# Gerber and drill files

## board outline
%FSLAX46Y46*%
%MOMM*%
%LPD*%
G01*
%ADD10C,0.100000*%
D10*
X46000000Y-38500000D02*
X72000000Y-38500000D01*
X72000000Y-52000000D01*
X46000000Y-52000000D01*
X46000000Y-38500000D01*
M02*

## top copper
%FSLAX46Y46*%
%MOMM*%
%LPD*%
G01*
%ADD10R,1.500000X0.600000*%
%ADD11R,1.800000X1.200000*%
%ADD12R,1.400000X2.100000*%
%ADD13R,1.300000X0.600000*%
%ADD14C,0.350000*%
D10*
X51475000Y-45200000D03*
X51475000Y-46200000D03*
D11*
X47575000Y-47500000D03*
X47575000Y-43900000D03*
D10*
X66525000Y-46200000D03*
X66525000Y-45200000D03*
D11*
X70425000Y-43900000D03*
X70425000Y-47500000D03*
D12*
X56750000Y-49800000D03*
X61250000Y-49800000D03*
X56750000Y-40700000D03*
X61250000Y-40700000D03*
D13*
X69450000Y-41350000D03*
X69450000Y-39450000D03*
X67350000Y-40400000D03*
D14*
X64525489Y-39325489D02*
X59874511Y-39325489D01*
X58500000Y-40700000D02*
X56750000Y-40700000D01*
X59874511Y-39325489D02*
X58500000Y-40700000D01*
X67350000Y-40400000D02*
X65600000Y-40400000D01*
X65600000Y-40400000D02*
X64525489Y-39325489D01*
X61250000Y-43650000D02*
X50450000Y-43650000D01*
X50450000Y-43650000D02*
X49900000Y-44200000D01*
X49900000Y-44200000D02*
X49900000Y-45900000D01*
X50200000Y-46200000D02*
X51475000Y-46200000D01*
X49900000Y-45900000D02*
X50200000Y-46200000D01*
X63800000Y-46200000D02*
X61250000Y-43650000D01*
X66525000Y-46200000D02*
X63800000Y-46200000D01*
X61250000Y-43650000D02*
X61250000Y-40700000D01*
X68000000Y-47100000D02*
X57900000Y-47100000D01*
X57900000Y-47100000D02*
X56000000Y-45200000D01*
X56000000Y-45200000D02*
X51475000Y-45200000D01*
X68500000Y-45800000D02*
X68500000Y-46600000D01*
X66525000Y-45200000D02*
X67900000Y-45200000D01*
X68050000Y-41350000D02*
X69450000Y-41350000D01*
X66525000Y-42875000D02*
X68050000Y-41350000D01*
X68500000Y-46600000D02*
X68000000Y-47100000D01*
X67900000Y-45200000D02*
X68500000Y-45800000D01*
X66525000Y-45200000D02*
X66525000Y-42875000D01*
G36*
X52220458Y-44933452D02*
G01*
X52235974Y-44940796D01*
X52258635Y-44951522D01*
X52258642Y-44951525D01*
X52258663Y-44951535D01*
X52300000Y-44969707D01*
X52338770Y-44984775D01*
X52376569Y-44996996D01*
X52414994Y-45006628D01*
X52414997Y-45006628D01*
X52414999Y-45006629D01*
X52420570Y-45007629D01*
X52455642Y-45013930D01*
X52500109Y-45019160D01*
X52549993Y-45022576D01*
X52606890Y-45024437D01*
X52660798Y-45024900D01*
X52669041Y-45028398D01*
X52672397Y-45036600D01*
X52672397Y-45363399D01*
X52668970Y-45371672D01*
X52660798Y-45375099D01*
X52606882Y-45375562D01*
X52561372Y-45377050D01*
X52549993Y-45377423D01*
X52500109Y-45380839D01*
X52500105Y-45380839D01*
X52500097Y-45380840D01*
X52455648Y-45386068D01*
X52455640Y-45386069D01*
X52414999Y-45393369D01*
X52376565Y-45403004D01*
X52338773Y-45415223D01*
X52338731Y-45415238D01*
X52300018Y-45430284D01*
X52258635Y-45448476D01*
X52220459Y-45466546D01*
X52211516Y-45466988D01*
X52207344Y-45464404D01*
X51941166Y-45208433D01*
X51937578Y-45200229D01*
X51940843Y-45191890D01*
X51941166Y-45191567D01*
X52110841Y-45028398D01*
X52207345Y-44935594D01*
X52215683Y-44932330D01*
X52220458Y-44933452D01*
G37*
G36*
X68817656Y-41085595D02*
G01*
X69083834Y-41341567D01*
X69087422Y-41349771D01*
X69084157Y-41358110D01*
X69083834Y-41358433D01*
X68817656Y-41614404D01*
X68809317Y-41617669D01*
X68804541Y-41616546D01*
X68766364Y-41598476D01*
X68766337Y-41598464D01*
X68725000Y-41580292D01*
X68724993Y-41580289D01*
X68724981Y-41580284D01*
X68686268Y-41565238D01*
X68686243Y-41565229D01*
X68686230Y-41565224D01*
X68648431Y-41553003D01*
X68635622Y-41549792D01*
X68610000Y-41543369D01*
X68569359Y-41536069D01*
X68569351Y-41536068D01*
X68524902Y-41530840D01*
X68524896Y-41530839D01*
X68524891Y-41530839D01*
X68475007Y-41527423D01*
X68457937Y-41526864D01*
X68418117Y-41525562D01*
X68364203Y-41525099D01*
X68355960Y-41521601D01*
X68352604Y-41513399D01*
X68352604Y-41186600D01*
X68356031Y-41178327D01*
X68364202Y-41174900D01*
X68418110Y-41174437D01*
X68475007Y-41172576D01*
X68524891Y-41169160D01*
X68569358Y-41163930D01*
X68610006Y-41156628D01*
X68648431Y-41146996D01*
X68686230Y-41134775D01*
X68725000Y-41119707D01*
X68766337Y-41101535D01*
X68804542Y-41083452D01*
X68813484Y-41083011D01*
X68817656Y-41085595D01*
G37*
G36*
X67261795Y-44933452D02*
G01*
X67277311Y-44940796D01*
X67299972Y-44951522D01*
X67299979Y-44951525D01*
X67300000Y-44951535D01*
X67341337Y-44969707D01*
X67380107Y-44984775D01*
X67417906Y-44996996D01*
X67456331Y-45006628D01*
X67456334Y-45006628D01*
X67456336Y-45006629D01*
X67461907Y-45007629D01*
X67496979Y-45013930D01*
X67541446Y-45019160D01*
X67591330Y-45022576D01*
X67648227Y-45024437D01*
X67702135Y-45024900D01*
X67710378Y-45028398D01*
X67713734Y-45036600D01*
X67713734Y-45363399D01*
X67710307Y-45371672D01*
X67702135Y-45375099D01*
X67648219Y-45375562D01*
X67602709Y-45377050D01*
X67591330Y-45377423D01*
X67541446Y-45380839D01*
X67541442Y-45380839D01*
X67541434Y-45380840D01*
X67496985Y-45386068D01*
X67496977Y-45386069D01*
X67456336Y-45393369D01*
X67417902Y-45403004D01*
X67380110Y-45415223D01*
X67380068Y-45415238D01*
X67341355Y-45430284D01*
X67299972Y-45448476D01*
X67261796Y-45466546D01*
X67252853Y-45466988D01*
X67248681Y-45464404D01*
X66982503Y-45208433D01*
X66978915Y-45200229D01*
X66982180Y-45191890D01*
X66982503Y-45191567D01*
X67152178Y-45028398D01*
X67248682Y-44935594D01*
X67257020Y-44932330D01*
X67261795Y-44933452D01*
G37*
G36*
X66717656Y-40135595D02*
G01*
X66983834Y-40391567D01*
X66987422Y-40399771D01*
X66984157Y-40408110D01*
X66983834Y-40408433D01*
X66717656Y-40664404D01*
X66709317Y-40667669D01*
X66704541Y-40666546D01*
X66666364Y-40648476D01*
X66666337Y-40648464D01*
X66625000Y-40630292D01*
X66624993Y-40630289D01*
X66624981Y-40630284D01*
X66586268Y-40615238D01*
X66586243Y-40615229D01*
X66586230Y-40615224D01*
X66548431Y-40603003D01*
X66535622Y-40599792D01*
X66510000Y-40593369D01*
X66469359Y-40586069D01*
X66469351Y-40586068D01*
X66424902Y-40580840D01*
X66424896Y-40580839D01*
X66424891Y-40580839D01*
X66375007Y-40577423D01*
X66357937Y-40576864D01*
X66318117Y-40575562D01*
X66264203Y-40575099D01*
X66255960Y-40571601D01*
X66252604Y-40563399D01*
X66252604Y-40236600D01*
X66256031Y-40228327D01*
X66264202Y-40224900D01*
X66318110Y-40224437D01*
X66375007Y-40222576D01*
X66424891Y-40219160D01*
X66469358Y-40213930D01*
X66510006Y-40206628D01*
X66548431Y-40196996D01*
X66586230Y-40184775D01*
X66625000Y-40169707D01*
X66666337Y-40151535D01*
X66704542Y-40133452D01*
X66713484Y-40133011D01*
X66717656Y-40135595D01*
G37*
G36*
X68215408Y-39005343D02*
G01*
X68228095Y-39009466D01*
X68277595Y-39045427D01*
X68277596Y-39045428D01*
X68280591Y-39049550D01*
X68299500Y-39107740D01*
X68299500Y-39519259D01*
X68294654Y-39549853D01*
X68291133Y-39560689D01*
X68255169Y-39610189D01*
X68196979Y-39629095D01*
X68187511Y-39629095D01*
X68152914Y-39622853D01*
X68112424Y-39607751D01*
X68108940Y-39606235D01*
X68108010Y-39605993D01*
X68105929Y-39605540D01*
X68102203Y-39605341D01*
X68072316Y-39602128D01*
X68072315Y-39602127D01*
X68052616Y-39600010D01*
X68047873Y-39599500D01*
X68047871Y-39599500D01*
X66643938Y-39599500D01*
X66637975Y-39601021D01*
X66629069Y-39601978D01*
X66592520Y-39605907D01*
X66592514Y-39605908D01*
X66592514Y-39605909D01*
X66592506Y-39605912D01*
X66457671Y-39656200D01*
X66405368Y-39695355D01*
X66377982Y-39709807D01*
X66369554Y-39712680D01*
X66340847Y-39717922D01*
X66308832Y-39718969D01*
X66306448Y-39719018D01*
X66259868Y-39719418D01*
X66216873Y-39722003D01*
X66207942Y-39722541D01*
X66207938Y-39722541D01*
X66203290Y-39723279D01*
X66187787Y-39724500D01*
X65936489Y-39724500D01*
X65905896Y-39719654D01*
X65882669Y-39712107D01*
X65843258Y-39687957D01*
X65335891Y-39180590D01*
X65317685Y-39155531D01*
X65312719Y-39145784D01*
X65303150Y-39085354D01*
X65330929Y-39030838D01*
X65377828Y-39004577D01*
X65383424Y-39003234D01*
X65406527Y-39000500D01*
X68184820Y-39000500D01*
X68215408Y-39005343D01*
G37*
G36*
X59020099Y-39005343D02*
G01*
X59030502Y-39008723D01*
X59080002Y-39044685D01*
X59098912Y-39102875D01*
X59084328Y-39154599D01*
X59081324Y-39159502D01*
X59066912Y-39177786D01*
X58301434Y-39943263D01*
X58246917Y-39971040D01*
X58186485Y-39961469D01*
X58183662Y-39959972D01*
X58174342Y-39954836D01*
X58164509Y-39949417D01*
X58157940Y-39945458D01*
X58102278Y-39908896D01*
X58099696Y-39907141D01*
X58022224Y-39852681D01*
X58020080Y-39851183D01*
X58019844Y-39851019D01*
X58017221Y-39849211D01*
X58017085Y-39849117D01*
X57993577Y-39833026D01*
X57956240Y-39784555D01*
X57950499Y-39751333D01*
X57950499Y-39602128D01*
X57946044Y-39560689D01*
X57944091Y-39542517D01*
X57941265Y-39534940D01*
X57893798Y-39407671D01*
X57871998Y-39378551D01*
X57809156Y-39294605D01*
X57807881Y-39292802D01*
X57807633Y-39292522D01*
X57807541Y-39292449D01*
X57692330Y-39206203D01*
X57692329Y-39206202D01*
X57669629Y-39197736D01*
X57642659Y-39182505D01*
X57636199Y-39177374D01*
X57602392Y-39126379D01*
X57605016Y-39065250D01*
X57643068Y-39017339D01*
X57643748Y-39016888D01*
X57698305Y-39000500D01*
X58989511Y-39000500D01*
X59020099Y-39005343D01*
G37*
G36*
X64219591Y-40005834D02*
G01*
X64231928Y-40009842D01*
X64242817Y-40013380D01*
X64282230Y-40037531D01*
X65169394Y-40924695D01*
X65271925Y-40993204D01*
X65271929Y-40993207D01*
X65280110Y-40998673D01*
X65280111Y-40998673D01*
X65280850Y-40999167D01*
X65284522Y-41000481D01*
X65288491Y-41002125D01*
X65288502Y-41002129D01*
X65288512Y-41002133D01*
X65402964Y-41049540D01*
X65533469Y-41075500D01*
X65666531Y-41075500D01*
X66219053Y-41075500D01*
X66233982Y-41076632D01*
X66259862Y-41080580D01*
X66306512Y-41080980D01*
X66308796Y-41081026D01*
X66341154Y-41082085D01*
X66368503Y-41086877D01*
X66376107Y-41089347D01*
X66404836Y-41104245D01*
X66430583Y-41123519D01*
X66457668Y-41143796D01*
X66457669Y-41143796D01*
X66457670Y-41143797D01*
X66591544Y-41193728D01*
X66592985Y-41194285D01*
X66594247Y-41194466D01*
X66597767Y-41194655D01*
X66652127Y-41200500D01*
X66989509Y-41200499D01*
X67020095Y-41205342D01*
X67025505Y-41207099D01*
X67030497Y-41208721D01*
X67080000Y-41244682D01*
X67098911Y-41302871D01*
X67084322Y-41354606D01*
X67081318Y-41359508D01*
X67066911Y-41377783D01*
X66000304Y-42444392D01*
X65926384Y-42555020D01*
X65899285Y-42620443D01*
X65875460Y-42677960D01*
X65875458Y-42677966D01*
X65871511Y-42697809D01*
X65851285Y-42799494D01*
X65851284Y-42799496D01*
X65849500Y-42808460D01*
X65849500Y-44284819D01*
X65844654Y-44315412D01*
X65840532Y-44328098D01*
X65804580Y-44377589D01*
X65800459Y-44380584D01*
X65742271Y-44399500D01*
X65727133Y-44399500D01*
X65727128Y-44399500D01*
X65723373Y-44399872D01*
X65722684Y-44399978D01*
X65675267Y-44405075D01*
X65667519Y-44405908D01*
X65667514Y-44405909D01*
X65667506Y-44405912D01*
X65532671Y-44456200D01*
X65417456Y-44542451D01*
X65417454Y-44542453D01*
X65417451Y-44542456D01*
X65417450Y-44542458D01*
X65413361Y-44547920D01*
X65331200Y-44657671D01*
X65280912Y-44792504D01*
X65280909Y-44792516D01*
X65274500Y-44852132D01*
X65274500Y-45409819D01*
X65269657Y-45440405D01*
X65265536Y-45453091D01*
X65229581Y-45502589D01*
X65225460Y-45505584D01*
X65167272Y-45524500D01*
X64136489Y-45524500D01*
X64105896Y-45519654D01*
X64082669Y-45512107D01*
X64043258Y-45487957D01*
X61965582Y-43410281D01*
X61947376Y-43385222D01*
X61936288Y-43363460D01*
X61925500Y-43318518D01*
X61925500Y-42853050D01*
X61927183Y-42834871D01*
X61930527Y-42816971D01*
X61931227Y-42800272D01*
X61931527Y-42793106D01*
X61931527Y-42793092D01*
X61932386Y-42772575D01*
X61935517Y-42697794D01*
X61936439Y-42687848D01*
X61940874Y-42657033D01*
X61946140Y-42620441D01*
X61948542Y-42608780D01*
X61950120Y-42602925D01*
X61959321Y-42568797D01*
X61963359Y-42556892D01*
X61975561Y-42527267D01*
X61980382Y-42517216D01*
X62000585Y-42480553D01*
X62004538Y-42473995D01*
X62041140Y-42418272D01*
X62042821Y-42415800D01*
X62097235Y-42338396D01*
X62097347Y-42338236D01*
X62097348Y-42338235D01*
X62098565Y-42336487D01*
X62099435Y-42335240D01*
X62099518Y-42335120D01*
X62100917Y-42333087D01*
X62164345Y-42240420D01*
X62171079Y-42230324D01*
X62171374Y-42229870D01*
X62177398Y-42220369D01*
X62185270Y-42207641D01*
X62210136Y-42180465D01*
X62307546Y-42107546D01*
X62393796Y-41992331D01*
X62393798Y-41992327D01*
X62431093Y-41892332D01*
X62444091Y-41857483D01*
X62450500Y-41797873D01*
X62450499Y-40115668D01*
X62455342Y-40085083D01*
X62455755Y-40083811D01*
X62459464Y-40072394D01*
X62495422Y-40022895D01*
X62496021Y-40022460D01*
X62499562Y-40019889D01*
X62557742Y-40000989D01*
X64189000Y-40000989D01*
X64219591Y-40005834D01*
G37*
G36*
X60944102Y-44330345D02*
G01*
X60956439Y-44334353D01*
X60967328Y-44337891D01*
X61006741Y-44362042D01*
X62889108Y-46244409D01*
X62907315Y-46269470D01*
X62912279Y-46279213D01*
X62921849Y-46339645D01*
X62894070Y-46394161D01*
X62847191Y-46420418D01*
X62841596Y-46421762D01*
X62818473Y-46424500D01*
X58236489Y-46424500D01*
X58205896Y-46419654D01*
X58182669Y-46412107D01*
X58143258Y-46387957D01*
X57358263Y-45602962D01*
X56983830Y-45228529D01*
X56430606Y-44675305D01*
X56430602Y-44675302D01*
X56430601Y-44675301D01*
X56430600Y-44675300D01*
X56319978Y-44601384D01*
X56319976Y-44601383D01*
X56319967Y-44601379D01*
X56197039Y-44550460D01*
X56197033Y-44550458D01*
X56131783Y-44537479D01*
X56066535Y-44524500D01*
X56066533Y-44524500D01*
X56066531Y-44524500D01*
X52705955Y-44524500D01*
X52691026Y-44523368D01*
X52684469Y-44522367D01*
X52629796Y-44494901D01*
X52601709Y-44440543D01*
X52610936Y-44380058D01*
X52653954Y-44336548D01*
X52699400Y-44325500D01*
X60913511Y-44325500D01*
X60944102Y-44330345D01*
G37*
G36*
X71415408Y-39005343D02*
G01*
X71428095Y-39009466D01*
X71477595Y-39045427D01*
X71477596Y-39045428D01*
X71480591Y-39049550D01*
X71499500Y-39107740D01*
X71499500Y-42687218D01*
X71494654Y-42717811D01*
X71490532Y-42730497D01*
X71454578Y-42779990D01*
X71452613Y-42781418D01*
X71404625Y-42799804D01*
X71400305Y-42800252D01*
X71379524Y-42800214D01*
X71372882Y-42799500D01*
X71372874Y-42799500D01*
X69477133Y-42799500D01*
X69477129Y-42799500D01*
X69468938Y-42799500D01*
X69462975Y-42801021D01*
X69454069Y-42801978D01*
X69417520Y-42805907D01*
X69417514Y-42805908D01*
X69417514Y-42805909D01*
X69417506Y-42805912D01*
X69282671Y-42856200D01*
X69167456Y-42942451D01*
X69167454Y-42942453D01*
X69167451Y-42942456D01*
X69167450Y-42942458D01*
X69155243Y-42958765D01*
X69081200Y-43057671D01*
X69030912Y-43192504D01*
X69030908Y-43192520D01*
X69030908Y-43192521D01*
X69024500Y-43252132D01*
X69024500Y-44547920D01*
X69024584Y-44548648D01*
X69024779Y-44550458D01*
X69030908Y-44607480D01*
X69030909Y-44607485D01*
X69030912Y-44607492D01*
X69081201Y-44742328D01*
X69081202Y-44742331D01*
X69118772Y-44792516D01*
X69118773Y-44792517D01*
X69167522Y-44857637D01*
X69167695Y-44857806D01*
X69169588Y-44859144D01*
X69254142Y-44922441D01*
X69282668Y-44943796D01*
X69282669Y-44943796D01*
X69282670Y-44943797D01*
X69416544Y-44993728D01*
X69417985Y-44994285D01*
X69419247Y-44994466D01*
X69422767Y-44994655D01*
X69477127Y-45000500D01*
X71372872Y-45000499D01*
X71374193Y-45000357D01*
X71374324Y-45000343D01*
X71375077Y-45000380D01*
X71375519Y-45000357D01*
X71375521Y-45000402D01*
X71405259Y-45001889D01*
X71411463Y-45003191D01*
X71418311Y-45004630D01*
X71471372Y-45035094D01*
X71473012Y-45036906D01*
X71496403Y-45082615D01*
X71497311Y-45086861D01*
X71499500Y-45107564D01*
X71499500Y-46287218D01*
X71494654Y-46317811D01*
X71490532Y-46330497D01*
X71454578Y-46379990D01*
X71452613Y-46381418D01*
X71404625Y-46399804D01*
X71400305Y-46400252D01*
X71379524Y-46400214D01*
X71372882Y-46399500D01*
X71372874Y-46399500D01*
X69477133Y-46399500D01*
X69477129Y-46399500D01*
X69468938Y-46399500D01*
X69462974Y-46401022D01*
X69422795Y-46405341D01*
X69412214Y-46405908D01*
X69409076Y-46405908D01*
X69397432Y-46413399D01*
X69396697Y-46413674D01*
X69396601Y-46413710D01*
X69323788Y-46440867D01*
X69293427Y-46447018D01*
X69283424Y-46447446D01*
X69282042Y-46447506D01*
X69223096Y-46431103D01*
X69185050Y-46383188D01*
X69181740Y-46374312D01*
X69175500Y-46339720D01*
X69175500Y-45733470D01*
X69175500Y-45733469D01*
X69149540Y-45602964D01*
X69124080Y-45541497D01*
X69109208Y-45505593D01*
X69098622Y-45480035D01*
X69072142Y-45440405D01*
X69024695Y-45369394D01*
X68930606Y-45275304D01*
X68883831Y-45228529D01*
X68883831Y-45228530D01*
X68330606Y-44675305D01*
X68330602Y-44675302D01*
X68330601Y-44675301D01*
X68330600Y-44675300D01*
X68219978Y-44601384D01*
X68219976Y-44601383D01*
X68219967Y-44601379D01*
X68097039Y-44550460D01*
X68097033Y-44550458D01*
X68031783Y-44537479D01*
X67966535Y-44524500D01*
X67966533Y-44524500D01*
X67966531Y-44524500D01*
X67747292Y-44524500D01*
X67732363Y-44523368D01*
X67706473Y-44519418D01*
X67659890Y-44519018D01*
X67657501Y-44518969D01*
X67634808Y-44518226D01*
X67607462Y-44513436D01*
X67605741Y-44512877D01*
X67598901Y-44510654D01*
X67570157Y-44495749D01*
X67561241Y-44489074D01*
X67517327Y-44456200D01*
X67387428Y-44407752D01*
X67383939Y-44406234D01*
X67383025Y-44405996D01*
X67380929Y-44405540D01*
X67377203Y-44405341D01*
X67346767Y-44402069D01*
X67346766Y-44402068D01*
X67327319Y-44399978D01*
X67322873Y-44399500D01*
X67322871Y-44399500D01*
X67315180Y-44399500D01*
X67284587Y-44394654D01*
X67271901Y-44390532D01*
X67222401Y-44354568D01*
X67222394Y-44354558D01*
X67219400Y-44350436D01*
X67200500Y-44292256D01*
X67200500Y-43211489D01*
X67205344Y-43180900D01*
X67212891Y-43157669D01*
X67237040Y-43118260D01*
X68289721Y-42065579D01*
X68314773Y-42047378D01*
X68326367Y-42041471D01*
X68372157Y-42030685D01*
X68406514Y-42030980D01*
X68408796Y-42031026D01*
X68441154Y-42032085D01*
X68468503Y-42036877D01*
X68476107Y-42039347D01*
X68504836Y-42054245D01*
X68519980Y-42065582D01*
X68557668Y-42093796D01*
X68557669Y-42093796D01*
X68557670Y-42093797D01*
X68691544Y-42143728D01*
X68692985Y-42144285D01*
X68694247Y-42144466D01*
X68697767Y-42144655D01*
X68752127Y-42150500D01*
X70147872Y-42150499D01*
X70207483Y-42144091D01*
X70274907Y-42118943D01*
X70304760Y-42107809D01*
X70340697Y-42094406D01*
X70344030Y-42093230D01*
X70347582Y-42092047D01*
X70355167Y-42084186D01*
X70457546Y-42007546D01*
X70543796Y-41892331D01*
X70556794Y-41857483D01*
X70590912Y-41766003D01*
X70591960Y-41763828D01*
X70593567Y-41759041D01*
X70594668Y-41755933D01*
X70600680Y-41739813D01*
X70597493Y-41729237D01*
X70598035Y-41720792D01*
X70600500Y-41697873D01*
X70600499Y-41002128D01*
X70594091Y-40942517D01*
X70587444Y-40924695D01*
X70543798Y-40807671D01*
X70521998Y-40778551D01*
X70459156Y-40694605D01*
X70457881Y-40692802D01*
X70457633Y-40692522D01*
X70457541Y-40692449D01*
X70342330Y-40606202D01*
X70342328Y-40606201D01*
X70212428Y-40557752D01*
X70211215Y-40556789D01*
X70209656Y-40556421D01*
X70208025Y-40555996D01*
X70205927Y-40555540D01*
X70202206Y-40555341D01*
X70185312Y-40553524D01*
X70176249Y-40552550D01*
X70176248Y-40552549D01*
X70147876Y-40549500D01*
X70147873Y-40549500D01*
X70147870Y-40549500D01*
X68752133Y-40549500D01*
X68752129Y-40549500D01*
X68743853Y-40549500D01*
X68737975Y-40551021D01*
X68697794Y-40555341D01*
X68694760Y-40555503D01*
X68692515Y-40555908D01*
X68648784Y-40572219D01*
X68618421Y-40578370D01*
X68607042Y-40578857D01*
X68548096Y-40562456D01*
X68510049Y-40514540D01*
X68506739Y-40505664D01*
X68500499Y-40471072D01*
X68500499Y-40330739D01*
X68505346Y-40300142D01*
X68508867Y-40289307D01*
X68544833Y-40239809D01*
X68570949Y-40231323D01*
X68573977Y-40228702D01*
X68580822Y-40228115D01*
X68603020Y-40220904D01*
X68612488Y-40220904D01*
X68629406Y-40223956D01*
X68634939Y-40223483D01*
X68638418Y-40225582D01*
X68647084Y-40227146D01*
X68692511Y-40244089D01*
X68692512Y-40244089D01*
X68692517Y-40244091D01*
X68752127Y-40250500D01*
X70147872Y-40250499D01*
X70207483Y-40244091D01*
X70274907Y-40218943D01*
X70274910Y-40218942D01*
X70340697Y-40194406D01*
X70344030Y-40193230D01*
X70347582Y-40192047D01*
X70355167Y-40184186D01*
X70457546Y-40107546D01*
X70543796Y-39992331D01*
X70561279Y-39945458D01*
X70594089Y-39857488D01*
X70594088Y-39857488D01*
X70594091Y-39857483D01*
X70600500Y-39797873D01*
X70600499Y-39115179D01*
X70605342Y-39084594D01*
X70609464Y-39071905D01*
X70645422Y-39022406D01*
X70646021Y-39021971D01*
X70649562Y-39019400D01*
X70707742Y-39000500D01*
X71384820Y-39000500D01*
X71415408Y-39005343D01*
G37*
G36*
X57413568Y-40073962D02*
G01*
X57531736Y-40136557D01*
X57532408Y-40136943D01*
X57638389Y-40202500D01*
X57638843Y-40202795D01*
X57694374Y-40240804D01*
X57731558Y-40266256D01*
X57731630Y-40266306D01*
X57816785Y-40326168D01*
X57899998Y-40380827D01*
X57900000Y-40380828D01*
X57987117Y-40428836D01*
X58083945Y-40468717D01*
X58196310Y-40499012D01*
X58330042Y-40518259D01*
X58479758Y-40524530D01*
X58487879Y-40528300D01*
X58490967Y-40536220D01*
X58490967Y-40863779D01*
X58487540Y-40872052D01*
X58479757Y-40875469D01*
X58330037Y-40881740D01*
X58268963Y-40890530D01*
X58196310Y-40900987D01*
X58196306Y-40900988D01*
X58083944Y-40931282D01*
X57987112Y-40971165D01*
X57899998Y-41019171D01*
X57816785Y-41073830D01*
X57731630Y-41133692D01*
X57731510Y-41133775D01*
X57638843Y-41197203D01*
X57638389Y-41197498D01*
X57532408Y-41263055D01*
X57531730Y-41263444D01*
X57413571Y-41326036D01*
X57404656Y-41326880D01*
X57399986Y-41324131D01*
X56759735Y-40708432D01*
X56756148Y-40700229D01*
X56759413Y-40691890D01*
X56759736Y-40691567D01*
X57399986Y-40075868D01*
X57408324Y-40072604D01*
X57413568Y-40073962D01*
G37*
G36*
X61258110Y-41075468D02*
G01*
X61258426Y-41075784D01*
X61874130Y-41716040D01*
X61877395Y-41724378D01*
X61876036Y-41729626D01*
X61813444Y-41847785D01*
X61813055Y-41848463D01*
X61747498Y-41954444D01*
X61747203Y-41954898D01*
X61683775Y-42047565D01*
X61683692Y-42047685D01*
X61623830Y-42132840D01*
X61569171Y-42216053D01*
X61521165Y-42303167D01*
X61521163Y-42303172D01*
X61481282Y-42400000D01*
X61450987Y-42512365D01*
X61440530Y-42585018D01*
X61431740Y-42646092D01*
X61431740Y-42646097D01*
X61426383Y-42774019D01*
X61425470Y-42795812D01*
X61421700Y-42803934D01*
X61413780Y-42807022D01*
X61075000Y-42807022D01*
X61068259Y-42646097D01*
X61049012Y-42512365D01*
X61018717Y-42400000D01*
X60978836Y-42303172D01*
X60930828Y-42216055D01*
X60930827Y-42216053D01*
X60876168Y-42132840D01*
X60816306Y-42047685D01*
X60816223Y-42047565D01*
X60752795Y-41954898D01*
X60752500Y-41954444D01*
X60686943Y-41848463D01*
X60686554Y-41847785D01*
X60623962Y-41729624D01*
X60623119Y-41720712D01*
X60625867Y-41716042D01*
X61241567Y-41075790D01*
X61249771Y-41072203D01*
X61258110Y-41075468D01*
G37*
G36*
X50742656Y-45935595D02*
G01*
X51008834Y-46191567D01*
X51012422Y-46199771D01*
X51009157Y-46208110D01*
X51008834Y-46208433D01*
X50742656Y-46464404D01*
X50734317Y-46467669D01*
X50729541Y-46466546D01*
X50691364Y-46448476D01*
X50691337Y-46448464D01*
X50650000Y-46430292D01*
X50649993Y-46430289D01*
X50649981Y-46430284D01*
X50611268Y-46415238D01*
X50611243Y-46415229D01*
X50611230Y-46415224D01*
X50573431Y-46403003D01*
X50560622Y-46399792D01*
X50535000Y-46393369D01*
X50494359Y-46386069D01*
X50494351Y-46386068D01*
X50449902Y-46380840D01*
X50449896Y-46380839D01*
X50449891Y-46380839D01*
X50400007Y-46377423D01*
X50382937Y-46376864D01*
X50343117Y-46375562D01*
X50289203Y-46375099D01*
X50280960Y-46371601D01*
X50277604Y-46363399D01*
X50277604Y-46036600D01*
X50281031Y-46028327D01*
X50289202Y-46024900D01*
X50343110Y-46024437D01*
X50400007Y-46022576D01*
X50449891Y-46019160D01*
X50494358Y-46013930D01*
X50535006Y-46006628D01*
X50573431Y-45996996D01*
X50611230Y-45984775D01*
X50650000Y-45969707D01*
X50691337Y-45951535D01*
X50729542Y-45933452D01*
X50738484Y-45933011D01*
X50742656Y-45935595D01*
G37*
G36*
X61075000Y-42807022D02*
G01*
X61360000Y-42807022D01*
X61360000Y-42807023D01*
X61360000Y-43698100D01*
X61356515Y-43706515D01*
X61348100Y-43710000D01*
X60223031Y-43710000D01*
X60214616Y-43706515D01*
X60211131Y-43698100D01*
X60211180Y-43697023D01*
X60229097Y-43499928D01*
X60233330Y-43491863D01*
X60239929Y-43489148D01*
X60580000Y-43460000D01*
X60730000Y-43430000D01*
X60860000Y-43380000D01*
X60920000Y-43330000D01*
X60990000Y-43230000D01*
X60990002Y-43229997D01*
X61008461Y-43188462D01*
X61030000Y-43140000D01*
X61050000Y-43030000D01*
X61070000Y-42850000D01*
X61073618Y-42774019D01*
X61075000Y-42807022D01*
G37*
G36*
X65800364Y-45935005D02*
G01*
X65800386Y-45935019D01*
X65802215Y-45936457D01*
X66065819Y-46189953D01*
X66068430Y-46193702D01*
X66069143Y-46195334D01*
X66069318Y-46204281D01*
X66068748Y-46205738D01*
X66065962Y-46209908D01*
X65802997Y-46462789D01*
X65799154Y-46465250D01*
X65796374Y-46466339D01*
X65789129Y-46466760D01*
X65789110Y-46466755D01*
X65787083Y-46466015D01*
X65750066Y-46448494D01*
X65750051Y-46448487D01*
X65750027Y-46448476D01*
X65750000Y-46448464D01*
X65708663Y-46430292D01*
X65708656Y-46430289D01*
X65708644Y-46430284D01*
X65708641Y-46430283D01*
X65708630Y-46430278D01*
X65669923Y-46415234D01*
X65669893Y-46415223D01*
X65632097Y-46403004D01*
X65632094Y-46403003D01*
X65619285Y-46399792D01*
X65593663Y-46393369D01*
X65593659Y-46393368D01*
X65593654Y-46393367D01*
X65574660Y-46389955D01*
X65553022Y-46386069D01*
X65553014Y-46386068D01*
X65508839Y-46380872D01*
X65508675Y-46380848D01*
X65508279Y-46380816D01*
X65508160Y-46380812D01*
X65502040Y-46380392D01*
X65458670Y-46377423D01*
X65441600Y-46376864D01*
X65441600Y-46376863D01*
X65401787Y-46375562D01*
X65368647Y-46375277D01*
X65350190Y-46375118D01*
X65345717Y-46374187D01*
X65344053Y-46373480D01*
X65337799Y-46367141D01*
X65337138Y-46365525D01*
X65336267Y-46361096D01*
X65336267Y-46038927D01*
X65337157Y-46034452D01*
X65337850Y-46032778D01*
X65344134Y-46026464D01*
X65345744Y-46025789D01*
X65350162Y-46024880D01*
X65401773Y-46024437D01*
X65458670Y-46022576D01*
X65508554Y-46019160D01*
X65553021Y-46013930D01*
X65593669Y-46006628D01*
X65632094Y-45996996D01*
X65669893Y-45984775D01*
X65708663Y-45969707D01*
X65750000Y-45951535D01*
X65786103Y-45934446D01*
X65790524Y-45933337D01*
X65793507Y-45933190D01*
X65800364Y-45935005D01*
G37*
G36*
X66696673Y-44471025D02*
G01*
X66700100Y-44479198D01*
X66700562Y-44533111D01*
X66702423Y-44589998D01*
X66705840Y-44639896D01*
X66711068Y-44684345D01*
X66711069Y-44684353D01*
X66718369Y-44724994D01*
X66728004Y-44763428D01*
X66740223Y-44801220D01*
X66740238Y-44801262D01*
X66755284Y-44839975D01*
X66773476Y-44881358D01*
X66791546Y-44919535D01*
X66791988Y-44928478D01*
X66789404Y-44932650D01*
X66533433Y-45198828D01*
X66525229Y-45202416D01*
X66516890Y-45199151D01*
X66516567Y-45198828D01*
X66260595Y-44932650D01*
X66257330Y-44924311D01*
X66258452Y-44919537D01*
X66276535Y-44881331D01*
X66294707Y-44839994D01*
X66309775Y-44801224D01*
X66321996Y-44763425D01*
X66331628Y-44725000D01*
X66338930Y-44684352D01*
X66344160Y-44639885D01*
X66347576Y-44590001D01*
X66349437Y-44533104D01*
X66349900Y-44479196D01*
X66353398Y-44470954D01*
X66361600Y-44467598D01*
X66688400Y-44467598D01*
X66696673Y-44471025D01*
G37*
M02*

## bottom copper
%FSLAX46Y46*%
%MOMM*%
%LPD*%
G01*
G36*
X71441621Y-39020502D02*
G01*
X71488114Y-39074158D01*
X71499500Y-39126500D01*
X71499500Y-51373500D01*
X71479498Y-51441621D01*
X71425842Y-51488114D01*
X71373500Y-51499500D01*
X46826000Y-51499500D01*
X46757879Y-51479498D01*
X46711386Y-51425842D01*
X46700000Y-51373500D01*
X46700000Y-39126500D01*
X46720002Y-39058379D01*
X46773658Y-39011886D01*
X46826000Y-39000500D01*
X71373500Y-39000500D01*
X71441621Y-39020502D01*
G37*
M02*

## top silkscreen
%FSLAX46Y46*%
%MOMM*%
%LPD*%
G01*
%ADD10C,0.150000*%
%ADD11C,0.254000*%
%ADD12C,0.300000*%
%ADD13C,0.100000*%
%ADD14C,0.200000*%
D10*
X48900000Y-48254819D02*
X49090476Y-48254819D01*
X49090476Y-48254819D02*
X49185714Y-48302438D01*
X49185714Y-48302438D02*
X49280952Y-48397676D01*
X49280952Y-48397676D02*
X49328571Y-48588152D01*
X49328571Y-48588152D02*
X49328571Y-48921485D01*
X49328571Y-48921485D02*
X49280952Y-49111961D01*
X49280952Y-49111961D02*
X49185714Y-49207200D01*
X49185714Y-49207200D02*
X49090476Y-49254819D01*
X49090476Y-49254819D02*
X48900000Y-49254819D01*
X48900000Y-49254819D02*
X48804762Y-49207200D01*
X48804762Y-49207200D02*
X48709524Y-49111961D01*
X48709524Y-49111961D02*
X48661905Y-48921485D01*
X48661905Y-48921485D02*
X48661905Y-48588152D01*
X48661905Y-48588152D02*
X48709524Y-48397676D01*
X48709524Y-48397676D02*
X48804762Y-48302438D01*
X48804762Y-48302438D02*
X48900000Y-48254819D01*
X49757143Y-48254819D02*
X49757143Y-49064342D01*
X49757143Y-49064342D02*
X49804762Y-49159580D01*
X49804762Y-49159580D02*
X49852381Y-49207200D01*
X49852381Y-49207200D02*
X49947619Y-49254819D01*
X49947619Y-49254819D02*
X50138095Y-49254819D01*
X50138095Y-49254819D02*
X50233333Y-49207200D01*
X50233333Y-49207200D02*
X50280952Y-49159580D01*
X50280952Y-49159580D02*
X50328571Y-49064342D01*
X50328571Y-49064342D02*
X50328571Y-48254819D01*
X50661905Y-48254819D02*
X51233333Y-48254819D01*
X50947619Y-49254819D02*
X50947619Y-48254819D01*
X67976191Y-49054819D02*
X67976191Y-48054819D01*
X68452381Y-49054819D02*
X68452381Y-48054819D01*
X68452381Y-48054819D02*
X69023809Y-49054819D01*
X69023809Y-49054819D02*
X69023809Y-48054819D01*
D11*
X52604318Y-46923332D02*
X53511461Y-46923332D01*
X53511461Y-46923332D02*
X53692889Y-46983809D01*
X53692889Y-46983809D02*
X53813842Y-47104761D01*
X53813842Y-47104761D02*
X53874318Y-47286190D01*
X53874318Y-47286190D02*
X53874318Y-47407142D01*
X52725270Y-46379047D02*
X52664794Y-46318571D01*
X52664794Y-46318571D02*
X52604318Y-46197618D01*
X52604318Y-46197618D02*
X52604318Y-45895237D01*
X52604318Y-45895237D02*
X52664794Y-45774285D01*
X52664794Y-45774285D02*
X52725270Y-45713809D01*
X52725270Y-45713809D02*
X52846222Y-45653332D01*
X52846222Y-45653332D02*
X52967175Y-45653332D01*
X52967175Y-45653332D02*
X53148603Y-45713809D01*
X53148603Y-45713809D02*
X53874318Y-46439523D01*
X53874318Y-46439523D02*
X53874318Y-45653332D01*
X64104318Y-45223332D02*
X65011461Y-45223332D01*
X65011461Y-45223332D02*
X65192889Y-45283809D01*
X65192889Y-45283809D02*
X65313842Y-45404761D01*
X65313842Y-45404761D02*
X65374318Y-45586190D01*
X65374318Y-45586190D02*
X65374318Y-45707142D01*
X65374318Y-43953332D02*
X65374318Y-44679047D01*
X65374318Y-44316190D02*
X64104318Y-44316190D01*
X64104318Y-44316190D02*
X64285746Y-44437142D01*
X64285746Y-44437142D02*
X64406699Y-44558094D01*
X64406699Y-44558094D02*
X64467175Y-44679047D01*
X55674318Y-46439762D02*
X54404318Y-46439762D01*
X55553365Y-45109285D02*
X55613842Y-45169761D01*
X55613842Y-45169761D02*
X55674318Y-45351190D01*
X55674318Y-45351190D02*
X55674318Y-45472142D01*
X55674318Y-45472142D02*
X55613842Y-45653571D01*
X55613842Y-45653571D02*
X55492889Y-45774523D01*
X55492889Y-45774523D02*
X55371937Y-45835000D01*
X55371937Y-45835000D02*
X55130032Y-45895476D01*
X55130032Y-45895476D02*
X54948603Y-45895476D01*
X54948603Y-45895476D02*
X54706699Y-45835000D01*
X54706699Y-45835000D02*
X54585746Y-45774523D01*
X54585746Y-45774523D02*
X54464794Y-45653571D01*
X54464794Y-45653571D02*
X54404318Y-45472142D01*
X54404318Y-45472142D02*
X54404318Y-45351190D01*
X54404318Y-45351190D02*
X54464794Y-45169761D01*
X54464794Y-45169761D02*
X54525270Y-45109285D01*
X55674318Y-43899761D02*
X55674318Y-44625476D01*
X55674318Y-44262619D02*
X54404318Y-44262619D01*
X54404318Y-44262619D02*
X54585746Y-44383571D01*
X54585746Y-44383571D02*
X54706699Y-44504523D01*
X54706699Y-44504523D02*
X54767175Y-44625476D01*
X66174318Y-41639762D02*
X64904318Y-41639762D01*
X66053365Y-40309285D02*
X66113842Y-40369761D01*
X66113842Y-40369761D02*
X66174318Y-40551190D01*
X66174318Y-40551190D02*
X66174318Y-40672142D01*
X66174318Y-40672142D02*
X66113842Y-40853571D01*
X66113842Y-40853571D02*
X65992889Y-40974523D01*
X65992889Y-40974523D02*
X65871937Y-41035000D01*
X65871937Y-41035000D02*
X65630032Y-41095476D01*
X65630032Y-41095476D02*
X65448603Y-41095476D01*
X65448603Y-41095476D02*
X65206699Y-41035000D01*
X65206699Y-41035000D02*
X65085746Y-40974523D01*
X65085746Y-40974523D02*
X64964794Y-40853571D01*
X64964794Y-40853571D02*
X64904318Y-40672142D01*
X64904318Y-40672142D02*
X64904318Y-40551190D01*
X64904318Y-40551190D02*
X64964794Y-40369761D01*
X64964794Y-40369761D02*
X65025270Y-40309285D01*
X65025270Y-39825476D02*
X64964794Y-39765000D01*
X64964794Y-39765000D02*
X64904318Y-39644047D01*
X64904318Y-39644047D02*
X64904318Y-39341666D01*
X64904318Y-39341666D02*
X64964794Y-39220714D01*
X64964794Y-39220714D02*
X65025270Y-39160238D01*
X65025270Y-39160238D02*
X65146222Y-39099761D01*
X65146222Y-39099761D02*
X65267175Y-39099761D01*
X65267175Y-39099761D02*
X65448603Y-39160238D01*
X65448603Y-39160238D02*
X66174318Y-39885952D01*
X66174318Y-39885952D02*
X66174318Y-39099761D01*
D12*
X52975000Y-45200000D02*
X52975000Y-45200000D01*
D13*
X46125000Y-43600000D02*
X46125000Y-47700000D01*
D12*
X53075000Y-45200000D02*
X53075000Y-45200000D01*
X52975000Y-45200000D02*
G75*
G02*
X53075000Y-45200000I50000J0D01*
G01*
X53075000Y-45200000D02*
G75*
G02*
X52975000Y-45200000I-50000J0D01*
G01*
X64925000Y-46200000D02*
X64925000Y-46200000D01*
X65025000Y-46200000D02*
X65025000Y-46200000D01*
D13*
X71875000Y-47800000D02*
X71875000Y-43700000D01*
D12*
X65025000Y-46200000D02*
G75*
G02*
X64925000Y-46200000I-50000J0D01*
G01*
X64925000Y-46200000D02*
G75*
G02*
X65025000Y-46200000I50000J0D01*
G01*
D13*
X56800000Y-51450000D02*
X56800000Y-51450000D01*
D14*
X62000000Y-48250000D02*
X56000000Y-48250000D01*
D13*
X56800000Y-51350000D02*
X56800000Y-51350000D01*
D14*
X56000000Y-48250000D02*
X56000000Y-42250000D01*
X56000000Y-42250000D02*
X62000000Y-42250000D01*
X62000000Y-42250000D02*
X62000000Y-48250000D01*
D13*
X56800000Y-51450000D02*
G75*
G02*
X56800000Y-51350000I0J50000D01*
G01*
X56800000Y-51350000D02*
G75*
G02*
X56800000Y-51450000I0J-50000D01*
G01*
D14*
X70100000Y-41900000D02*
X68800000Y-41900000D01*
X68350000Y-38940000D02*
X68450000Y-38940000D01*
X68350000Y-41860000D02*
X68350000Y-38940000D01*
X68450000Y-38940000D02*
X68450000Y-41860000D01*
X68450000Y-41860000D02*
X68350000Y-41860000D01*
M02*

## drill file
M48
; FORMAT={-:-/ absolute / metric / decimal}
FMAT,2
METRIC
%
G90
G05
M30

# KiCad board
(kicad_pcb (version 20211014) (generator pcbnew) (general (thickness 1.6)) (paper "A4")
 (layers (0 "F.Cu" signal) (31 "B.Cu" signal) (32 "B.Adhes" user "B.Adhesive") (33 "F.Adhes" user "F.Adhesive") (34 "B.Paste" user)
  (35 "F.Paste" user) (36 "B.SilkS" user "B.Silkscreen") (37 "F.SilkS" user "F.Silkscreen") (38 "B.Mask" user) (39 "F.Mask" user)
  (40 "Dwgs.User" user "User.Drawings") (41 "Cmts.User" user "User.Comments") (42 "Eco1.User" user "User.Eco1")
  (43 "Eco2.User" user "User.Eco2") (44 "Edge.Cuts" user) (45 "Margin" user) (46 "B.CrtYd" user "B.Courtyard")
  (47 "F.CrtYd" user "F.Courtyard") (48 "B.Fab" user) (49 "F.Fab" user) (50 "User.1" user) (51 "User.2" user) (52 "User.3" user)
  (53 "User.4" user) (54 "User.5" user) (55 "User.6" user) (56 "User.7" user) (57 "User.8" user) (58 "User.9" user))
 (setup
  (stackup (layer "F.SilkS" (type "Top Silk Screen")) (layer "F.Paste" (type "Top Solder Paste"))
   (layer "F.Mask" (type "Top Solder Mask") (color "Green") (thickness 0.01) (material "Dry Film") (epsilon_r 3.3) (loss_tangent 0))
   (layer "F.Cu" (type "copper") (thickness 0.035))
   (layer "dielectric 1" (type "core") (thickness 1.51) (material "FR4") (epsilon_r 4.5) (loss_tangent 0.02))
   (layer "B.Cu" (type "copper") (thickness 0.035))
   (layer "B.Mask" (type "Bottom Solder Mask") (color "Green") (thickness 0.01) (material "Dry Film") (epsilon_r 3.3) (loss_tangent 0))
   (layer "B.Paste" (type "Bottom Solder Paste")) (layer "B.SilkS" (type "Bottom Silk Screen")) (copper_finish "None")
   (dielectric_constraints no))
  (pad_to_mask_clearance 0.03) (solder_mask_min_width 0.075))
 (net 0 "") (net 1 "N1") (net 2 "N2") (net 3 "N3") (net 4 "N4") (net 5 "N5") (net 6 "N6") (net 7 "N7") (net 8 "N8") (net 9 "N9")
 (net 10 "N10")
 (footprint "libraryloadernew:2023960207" (layer "F.Cu") (at 49.6 45.65 -90)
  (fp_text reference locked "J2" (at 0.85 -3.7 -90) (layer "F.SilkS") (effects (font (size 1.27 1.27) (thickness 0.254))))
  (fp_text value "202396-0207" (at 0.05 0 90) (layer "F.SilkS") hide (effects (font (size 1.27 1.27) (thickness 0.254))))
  (fp_line (start -0.45 -3.375) (end -0.45 -3.375) (layer "F.SilkS") (width 0.3))
  (fp_line (start -2.05 3.475) (end 2.05 3.475) (layer "F.SilkS") (width 0.1))
  (fp_line (start -0.45 -3.475) (end -0.45 -3.475) (layer "F.SilkS") (width 0.3))
  (fp_arc (start -0.45 -3.375) (mid -0.5 -3.425) (end -0.45 -3.475) (layer "F.SilkS") (width 0.3))
  (fp_arc (start -0.45 -3.475) (mid -0.4 -3.425) (end -0.45 -3.375) (layer "F.SilkS") (width 0.3))
  (pad "1" smd rect locked (at -0.45 -1.875 270) (size 0.6 1.5) (layers "F.Cu" "F.Paste" "F.Mask") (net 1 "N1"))
  (pad "2" smd rect locked (at 0.55 -1.875 270) (size 0.6 1.5) (layers "F.Cu" "F.Paste" "F.Mask") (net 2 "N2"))
  (pad "MP1" smd rect locked (at 1.85 2.025 270) (size 1.2 1.8) (layers "F.Cu" "F.Paste" "F.Mask") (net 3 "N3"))
  (pad "MP2" smd rect locked (at -1.75 2.025 270) (size 1.2 1.8) (layers "F.Cu" "F.Paste" "F.Mask") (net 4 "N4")))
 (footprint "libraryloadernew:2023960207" (layer "F.Cu") (at 68.4 45.75 90)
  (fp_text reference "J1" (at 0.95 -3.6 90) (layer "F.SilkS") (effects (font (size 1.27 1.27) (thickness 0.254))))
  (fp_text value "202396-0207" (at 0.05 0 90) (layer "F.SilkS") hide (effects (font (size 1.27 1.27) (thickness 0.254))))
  (fp_line (start -0.45 -3.475) (end -0.45 -3.475) (layer "F.SilkS") (width 0.3))
  (fp_line (start -0.45 -3.375) (end -0.45 -3.375) (layer "F.SilkS") (width 0.3))
  (fp_line (start -2.05 3.475) (end 2.05 3.475) (layer "F.SilkS") (width 0.1))
  (fp_arc (start -0.45 -3.375) (mid -0.5 -3.425) (end -0.45 -3.475) (layer "F.SilkS") (width 0.3))
  (fp_arc (start -0.45 -3.475) (mid -0.4 -3.425) (end -0.45 -3.375) (layer "F.SilkS") (width 0.3))
  (pad "1" smd rect locked (at -0.45 -1.875 90) (size 0.6 1.5) (layers "F.Cu" "F.Paste" "F.Mask") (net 2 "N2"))
  (pad "2" smd rect locked (at 0.55 -1.875 90) (size 0.6 1.5) (layers "F.Cu" "F.Paste" "F.Mask") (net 1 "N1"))
  (pad "MP1" smd rect locked (at 1.85 2.025 90) (size 1.2 1.8) (layers "F.Cu" "F.Paste" "F.Mask") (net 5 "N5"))
  (pad "MP2" smd rect locked (at -1.75 2.025 90) (size 1.2 1.8) (layers "F.Cu" "F.Paste" "F.Mask") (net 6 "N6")))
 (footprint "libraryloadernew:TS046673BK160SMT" (layer "F.Cu") (at 59 45.25 90)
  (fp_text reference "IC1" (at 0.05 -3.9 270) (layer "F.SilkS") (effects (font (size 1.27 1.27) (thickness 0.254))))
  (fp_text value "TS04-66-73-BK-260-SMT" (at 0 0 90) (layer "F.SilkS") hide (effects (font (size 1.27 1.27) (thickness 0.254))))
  (fp_line (start -6.2 -2.2) (end -6.2 -2.2) (layer "F.SilkS") (width 0.1))
  (fp_line (start -3 3) (end -3 -3) (layer "F.SilkS") (width 0.2))
  (fp_line (start -6.1 -2.2) (end -6.1 -2.2) (layer "F.SilkS") (width 0.1))
  (fp_line (start -3 -3) (end 3 -3) (layer "F.SilkS") (width 0.2))
  (fp_line (start 3 -3) (end 3 3) (layer "F.SilkS") (width 0.2))
  (fp_line (start 3 3) (end -3 3) (layer "F.SilkS") (width 0.2))
  (fp_arc (start -6.2 -2.2) (mid -6.15 -2.25) (end -6.1 -2.2) (layer "F.SilkS") (width 0.1))
  (fp_arc (start -6.1 -2.2) (mid -6.15 -2.15) (end -6.2 -2.2) (layer "F.SilkS") (width 0.1))
  (pad "1" smd rect locked (at -4.55 -2.25 180) (size 1.4 2.1) (layers "F.Cu" "F.Paste" "F.Mask") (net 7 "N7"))
  (pad "2" smd rect locked (at -4.55 2.25 180) (size 1.4 2.1) (layers "F.Cu" "F.Paste" "F.Mask") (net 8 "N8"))
  (pad "3" smd rect locked (at 4.55 -2.25 180) (size 1.4 2.1) (layers "F.Cu" "F.Paste" "F.Mask") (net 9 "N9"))
  (pad "4" smd rect locked (at 4.55 2.25 180) (size 1.4 2.1) (layers "F.Cu" "F.Paste" "F.Mask") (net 2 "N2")))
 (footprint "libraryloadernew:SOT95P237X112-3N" (layer "F.Cu") (at 68.4 40.4 180)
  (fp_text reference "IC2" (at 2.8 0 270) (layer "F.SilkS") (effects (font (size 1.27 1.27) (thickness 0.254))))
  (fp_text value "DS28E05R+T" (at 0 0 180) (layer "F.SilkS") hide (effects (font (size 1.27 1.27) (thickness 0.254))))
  (fp_line (start -1.7 -1.5) (end -0.4 -1.5) (layer "F.SilkS") (width 0.2))
  (fp_line (start 0.05 1.46) (end -0.05 1.46) (layer "F.SilkS") (width 0.2))
  (fp_line (start 0.05 -1.46) (end 0.05 1.46) (layer "F.SilkS") (width 0.2))
  (fp_line (start -0.05 1.46) (end -0.05 -1.46) (layer "F.SilkS") (width 0.2))
  (fp_line (start -0.05 -1.46) (end 0.05 -1.46) (layer "F.SilkS") (width 0.2))
  (pad "1" smd rect locked (at -1.05 -0.95 270) (size 0.6 1.3) (layers "F.Cu" "F.Paste" "F.Mask") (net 1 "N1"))
  (pad "2" smd rect locked (at -1.05 0.95 270) (size 0.6 1.3) (layers "F.Cu" "F.Paste" "F.Mask") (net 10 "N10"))
  (pad "3" smd rect locked (at 1.05 0 270) (size 0.6 1.3) (layers "F.Cu" "F.Paste" "F.Mask") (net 9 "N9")))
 (gr_rect (start 46 38.5) (end 72 52) (layer "Edge.Cuts") (width 0.1) (fill none))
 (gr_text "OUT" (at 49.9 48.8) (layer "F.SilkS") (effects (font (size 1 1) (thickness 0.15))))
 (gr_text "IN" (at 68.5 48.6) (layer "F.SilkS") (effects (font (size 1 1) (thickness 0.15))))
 (segment (start 64.525489 39.325489) (end 59.874511 39.325489) (width 0.35) (layer "F.Cu") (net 9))
 (segment (start 58.5 40.7) (end 56.75 40.7) (width 0.35) (layer "F.Cu") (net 9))
 (segment (start 59.874511 39.325489) (end 58.5 40.7) (width 0.35) (layer "F.Cu") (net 9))
 (segment (start 67.35 40.4) (end 65.6 40.4) (width 0.35) (layer "F.Cu") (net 9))
 (segment (start 65.6 40.4) (end 64.525489 39.325489) (width 0.35) (layer "F.Cu") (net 9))
 (segment (start 61.25 43.65) (end 50.45 43.65) (width 0.35) (layer "F.Cu") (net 2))
 (segment (start 50.45 43.65) (end 49.9 44.2) (width 0.35) (layer "F.Cu") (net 2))
 (segment (start 49.9 44.2) (end 49.9 45.9) (width 0.35) (layer "F.Cu") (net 2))
 (segment (start 50.2 46.2) (end 51.475 46.2) (width 0.35) (layer "F.Cu") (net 2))
 (segment (start 49.9 45.9) (end 50.2 46.2) (width 0.35) (layer "F.Cu") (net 2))
 (segment (start 63.8 46.2) (end 61.25 43.65) (width 0.35) (layer "F.Cu") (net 2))
 (segment (start 66.525 46.2) (end 63.8 46.2) (width 0.35) (layer "F.Cu") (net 2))
 (segment (start 61.25 43.65) (end 61.25 40.7) (width 0.35) (layer "F.Cu") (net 2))
 (segment (start 68 47.1) (end 57.9 47.1) (width 0.35) (layer "F.Cu") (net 1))
 (segment (start 57.9 47.1) (end 56 45.2) (width 0.35) (layer "F.Cu") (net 1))
 (segment (start 56 45.2) (end 51.475 45.2) (width 0.35) (layer "F.Cu") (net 1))
 (segment (start 68.5 45.8) (end 68.5 46.6) (width 0.35) (layer "F.Cu") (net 1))
 (segment (start 66.525 45.2) (end 67.9 45.2) (width 0.35) (layer "F.Cu") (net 1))
 (segment (start 68.05 41.35) (end 69.45 41.35) (width 0.35) (layer "F.Cu") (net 1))
 (segment (start 66.525 42.875) (end 68.05 41.35) (width 0.35) (layer "F.Cu") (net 1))
 (segment (start 68.5 46.6) (end 68 47.1) (width 0.35) (layer "F.Cu") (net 1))
 (segment (start 67.9 45.2) (end 68.5 45.8) (width 0.35) (layer "F.Cu") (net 1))
 (segment (start 66.525 45.2) (end 66.525 42.875) (width 0.35) (layer "F.Cu") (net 1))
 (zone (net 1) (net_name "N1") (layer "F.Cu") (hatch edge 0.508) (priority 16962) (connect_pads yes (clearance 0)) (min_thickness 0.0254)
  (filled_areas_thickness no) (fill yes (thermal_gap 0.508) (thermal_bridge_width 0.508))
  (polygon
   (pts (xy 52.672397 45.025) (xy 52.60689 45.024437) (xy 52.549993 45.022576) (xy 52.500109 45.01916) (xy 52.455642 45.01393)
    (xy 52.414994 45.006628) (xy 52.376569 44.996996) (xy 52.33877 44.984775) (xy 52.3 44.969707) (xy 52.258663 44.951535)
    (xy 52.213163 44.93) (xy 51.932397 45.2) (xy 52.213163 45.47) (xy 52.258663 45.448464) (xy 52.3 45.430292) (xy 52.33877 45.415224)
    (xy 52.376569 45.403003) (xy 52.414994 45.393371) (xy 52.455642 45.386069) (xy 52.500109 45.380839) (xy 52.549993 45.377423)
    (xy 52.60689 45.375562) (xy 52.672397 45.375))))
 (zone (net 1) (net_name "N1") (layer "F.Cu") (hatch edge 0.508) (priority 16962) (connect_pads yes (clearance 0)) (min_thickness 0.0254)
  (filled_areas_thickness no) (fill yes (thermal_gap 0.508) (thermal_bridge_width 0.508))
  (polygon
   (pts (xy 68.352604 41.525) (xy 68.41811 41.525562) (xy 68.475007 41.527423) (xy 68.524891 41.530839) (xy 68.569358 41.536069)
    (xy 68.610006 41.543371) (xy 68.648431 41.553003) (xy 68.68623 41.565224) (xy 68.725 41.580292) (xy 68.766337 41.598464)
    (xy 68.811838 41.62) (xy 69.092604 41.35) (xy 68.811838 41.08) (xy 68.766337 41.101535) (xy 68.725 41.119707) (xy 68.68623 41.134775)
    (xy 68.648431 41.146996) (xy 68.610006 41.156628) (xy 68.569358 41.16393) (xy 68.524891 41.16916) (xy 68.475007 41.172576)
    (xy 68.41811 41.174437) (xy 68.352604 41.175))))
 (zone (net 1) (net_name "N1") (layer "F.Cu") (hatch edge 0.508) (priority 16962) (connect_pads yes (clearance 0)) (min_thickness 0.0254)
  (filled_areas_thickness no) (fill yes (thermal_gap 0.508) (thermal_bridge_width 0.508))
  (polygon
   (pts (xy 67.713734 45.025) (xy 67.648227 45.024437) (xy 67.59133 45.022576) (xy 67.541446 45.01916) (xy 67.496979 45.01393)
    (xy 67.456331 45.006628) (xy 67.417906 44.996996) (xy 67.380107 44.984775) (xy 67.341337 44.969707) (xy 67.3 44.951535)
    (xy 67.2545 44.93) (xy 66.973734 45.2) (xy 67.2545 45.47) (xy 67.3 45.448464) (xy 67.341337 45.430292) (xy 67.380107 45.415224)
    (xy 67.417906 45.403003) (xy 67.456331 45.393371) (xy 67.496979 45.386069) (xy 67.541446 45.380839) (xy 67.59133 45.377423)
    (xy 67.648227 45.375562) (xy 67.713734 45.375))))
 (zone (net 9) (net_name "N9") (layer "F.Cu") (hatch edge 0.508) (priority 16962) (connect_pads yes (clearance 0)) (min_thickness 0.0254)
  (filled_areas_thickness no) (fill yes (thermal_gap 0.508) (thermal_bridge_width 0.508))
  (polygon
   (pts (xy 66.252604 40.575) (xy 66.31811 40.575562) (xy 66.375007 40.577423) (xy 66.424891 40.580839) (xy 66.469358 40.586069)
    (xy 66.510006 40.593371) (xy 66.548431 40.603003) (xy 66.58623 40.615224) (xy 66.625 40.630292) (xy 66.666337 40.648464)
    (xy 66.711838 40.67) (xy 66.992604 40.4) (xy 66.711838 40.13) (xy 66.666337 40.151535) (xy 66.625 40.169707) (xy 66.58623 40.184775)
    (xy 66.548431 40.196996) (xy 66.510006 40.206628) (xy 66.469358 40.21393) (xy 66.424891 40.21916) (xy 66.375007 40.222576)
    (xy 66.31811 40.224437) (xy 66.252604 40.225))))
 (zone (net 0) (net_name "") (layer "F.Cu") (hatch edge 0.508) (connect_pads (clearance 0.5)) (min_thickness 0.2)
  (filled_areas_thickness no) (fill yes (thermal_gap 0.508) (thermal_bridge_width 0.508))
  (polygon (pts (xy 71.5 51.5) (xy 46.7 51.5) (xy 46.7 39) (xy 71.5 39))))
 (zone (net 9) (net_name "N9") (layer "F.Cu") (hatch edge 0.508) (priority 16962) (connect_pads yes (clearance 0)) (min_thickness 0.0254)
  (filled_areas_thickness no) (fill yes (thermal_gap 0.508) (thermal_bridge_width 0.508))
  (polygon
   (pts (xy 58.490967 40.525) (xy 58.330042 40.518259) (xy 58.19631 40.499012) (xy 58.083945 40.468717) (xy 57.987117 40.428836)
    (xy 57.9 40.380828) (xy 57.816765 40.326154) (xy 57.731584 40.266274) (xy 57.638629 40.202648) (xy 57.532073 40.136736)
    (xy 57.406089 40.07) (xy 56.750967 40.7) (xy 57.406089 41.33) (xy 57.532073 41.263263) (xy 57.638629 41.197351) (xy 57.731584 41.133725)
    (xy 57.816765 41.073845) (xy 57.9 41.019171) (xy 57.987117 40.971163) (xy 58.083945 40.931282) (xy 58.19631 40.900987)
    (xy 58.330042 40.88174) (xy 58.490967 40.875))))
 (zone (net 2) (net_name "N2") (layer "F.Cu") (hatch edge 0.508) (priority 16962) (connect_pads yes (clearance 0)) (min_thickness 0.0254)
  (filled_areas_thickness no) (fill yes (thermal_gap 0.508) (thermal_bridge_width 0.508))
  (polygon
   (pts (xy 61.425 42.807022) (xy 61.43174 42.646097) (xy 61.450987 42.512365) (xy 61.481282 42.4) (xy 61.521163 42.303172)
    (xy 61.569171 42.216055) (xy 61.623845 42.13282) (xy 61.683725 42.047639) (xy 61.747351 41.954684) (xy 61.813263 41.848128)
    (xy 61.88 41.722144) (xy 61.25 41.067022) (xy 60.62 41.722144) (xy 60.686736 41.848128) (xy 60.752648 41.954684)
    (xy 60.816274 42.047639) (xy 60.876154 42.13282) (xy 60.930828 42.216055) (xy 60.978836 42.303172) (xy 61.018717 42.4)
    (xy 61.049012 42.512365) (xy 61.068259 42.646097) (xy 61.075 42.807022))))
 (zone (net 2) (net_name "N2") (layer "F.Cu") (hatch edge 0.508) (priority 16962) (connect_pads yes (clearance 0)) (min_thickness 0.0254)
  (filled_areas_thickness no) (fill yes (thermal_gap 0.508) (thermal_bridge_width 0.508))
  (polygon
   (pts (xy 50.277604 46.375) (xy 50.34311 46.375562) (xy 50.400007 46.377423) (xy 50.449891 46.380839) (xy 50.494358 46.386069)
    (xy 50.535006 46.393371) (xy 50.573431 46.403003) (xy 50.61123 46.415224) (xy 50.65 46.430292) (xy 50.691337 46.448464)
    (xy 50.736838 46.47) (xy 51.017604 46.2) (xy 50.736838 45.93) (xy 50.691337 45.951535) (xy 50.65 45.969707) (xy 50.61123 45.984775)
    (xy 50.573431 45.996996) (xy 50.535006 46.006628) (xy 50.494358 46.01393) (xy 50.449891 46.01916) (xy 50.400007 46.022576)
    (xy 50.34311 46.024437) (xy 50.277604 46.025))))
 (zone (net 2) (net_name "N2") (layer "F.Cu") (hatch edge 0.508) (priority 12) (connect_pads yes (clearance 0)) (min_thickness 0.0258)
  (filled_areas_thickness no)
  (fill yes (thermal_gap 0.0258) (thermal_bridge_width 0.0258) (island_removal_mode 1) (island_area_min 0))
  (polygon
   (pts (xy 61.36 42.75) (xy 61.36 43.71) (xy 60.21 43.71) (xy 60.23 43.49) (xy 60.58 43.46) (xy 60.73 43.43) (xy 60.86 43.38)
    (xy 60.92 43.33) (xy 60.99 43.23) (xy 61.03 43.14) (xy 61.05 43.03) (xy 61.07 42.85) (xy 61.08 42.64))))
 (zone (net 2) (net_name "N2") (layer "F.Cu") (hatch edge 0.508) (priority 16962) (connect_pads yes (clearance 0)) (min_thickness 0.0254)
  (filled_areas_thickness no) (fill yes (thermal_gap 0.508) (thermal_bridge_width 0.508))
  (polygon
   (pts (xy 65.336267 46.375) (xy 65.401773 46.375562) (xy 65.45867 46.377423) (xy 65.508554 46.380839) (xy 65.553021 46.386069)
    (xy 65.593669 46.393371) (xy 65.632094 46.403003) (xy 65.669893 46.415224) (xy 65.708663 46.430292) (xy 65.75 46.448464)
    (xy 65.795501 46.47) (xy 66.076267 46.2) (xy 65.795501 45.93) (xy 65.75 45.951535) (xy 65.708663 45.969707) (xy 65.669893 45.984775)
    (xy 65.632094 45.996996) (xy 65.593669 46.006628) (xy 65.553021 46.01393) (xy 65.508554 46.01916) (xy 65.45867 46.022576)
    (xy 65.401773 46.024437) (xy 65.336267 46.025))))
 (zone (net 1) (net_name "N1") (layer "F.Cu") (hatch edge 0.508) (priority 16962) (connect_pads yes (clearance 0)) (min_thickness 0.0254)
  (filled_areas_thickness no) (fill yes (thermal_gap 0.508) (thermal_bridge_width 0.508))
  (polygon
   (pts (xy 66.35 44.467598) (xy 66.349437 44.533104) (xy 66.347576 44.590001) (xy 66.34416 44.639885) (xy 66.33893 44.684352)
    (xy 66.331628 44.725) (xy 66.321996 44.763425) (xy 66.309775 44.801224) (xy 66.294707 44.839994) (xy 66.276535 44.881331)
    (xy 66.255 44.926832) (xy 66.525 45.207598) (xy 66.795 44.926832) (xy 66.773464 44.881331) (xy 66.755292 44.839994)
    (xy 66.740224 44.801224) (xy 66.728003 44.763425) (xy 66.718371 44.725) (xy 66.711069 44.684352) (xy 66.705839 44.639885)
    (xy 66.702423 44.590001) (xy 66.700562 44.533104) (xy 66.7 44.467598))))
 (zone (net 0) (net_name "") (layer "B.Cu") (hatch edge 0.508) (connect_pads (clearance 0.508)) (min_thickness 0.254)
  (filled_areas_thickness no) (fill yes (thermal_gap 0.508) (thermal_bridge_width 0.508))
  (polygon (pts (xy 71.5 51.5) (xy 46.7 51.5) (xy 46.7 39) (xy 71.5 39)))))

